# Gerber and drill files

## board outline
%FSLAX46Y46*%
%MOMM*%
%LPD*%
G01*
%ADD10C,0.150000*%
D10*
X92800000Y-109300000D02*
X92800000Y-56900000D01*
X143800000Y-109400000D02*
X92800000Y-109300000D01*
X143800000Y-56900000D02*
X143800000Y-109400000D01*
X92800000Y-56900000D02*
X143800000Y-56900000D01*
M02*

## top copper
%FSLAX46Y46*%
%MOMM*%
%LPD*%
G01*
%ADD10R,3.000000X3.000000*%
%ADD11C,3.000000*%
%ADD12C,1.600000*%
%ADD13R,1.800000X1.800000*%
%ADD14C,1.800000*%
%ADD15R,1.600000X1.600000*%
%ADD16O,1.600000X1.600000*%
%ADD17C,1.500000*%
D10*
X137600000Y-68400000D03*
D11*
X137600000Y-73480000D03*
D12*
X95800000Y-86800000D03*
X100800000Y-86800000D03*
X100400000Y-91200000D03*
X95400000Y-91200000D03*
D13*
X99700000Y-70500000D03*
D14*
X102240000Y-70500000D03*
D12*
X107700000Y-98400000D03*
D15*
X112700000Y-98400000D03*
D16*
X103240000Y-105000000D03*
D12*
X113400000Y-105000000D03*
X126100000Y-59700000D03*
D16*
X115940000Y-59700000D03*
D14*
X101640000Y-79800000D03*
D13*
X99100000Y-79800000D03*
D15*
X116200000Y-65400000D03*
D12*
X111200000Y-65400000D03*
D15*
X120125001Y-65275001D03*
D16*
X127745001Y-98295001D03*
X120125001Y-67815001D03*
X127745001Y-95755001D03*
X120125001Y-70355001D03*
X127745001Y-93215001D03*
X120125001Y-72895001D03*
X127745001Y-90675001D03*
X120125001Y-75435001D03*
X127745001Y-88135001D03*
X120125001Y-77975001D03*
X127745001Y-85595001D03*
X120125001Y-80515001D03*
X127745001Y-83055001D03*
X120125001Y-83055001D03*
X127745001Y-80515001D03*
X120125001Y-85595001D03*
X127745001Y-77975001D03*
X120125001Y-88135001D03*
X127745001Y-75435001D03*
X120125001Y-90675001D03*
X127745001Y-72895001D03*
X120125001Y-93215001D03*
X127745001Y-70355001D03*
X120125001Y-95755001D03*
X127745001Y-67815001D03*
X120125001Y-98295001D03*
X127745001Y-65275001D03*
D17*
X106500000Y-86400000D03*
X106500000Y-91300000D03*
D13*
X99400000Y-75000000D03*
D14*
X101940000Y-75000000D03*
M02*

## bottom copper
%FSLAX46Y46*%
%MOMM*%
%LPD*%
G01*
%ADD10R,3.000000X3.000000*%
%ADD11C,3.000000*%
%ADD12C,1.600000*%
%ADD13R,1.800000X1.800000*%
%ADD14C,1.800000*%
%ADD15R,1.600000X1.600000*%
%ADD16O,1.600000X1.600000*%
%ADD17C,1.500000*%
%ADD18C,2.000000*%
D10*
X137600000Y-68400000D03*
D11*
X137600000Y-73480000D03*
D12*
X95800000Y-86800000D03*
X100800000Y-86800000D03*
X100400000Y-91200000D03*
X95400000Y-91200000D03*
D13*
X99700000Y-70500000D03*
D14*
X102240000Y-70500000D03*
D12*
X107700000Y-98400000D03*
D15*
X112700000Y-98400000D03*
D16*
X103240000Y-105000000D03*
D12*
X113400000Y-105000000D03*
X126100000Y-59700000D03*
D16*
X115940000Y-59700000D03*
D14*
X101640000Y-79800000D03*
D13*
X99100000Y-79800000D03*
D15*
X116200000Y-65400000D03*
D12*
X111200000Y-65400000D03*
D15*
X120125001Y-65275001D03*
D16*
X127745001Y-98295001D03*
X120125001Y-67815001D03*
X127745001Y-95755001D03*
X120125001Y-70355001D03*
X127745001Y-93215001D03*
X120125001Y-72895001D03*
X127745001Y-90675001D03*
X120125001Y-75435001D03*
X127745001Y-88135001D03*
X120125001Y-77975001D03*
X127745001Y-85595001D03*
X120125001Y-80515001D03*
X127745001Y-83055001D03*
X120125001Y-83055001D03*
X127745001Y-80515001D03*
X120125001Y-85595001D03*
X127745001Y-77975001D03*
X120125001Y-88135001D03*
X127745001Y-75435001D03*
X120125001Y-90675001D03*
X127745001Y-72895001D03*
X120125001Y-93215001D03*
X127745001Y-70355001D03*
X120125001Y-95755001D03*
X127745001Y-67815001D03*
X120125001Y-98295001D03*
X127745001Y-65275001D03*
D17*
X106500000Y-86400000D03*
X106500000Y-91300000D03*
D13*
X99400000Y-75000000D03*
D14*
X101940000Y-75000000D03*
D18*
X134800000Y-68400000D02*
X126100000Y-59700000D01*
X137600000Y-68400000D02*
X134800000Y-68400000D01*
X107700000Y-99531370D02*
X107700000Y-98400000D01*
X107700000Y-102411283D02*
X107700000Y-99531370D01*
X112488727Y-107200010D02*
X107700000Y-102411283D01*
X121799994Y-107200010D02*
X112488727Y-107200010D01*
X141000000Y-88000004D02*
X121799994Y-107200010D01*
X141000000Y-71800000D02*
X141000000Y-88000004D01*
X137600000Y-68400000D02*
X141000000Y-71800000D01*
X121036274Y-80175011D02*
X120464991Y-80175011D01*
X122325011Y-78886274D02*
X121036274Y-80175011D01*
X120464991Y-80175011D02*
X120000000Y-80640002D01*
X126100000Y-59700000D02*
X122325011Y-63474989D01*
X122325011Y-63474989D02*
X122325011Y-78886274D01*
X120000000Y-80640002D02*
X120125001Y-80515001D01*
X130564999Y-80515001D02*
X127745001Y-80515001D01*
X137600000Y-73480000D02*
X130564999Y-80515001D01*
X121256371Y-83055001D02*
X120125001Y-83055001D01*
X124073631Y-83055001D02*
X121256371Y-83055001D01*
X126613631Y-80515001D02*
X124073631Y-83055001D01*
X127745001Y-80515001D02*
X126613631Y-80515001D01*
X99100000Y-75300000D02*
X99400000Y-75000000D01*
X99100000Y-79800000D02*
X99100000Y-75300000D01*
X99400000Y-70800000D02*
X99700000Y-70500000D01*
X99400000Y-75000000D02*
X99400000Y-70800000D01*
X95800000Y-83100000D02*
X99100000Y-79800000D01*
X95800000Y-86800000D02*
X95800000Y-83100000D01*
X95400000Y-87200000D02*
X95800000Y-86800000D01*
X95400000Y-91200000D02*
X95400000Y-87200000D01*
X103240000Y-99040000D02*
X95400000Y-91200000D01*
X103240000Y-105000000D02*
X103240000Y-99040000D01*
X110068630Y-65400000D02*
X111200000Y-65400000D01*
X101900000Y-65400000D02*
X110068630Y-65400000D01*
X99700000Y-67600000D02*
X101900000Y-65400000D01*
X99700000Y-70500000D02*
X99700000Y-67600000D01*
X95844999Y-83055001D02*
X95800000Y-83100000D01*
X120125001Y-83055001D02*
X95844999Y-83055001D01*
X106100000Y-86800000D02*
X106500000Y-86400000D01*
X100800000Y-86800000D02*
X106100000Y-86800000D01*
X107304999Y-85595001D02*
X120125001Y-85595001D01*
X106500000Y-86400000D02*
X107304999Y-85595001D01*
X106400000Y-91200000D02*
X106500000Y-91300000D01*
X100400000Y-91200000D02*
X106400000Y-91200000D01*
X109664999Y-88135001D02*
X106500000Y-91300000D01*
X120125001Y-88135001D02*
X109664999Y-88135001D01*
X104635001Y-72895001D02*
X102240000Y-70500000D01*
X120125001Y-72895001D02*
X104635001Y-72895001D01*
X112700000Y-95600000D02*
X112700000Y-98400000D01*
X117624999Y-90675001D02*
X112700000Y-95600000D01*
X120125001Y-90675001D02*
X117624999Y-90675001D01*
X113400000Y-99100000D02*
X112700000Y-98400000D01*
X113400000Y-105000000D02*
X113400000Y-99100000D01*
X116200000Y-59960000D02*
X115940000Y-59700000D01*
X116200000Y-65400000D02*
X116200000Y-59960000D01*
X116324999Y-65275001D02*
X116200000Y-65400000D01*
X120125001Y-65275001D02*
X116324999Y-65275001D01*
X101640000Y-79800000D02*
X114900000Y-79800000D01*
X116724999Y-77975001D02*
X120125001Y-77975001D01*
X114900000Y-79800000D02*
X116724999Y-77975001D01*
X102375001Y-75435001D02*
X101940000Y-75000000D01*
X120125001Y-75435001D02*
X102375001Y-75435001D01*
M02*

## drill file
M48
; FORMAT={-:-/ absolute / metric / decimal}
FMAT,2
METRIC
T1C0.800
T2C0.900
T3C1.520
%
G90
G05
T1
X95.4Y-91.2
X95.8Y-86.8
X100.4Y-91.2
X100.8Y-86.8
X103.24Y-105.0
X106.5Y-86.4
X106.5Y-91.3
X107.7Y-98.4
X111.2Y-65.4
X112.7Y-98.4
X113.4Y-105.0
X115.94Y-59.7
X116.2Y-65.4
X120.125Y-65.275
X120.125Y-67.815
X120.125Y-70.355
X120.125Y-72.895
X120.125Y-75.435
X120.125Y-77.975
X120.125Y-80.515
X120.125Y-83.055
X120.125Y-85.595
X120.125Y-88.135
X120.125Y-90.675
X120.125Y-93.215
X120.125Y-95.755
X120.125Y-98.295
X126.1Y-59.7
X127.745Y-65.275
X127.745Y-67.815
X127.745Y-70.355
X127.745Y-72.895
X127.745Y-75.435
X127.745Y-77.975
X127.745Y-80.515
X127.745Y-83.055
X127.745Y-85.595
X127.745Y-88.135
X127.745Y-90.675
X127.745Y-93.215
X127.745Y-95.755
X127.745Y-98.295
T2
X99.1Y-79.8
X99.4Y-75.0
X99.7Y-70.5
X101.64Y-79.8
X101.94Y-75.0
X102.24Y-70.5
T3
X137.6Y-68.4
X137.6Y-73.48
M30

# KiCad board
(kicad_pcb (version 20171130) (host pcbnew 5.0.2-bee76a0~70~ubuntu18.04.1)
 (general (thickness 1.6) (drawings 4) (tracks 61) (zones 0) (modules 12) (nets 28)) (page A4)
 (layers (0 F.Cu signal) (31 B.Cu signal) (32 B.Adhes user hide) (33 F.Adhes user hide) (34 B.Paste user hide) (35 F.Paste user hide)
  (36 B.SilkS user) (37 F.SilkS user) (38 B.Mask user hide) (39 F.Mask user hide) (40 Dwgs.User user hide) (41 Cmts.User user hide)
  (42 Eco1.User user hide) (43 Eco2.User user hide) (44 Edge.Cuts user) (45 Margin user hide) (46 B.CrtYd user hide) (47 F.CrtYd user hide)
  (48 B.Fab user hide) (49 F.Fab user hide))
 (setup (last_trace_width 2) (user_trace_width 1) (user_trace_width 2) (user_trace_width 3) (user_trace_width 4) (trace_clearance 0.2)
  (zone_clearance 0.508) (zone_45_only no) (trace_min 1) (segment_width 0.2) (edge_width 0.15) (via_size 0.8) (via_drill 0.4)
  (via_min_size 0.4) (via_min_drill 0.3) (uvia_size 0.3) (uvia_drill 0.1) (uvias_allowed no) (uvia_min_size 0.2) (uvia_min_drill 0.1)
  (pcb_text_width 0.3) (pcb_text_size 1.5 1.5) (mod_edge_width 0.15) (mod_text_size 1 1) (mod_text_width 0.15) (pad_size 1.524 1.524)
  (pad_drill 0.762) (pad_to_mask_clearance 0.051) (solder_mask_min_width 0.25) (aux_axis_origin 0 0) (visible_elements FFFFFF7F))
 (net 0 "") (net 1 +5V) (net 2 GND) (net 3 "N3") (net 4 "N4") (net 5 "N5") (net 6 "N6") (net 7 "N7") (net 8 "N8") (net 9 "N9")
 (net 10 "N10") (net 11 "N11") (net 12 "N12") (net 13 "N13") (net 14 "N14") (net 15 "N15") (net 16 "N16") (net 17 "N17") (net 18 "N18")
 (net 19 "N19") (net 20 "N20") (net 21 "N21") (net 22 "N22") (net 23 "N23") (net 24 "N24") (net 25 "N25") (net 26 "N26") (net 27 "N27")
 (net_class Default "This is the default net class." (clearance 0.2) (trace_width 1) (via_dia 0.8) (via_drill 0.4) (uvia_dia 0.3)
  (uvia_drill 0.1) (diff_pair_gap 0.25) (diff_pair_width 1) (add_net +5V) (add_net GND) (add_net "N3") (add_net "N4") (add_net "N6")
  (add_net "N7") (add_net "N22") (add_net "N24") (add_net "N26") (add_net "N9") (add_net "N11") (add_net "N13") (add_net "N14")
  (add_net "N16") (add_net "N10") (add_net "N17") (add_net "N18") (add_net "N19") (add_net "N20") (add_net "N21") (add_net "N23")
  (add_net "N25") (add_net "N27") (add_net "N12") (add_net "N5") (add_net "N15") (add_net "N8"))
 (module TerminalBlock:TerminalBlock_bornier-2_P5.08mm (layer F.Cu) (at 137.6 68.4 270)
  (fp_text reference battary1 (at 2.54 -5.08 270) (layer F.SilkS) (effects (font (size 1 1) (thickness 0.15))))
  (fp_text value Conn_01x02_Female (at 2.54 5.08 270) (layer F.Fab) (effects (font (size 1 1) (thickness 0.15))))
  (pad 1 thru_hole rect (at 0 0 270) (size 3 3) (drill 1.52) (layers *.Cu *.Mask) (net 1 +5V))
  (pad 2 thru_hole circle (at 5.08 0 270) (size 3 3) (drill 1.52) (layers *.Cu *.Mask) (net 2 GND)))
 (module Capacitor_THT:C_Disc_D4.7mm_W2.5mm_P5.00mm (layer F.Cu) (at 95.8 86.8)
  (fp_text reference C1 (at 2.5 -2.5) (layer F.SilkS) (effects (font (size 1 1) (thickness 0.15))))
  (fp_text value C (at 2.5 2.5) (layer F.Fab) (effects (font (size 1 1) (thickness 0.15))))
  (pad 1 thru_hole circle (at 0 0) (size 1.6 1.6) (drill 0.8) (layers *.Cu *.Mask) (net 2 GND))
  (pad 2 thru_hole circle (at 5 0) (size 1.6 1.6) (drill 0.8) (layers *.Cu *.Mask) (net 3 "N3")))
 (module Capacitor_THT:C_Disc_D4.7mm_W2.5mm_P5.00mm (layer F.Cu) (at 95.4 91.2)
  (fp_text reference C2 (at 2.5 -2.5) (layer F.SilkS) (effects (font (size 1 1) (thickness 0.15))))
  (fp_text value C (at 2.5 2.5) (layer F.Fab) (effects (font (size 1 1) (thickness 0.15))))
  (pad 2 thru_hole circle (at 5 0) (size 1.6 1.6) (drill 0.8) (layers *.Cu *.Mask) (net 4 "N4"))
  (pad 1 thru_hole circle (at 0 0) (size 1.6 1.6) (drill 0.8) (layers *.Cu *.Mask) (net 2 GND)))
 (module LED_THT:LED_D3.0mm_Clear (layer F.Cu) (at 99.7 70.5)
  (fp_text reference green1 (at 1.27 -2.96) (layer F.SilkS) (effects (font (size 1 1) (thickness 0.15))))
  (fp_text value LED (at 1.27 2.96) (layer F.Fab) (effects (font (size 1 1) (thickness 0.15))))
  (pad 1 thru_hole rect (at 0 0) (size 1.8 1.8) (drill 0.9) (layers *.Cu *.Mask) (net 2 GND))
  (pad 2 thru_hole circle (at 2.54 0) (size 1.8 1.8) (drill 0.9) (layers *.Cu *.Mask) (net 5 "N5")))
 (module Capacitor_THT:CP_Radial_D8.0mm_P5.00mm (layer F.Cu) (at 112.7 98.4 180)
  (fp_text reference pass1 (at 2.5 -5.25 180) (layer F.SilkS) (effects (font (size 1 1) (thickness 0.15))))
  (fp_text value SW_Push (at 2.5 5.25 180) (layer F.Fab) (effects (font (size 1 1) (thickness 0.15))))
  (pad 2 thru_hole circle (at 5 0 180) (size 1.6 1.6) (drill 0.8) (layers *.Cu *.Mask) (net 1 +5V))
  (pad 1 thru_hole rect (at 0 0 180) (size 1.6 1.6) (drill 0.8) (layers *.Cu *.Mask) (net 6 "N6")))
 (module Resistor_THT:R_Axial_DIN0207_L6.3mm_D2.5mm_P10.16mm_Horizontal (layer F.Cu) (at 113.4 105 180)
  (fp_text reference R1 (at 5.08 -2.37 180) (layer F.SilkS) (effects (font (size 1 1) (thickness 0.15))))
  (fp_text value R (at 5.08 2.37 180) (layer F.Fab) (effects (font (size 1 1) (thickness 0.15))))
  (pad 2 thru_hole oval (at 10.16 0 180) (size 1.6 1.6) (drill 0.8) (layers *.Cu *.Mask) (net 2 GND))
  (pad 1 thru_hole circle (at 0 0 180) (size 1.6 1.6) (drill 0.8) (layers *.Cu *.Mask) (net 6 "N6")))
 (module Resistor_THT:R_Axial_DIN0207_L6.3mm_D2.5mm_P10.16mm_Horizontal (layer F.Cu) (at 126.1 59.7 180)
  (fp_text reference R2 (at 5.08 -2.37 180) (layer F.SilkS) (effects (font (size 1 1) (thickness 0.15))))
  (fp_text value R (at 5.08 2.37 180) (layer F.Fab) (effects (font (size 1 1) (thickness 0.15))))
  (pad 1 thru_hole circle (at 0 0 180) (size 1.6 1.6) (drill 0.8) (layers *.Cu *.Mask) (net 1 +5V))
  (pad 2 thru_hole oval (at 10.16 0 180) (size 1.6 1.6) (drill 0.8) (layers *.Cu *.Mask) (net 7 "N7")))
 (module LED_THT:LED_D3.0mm (layer F.Cu) (at 99.1 79.8)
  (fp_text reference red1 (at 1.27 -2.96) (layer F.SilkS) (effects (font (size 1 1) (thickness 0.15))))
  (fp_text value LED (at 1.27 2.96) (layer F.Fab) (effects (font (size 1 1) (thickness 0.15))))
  (pad 2 thru_hole circle (at 2.54 0) (size 1.8 1.8) (drill 0.9) (layers *.Cu *.Mask) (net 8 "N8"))
  (pad 1 thru_hole rect (at 0 0) (size 1.8 1.8) (drill 0.9) (layers *.Cu *.Mask) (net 2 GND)))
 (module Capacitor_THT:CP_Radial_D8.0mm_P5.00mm (layer F.Cu) (at 116.2 65.4 180)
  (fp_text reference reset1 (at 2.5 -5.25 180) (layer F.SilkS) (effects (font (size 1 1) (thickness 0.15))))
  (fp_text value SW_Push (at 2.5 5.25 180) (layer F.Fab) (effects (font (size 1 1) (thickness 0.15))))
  (pad 1 thru_hole rect (at 0 0 180) (size 1.6 1.6) (drill 0.8) (layers *.Cu *.Mask) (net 7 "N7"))
  (pad 2 thru_hole circle (at 5 0 180) (size 1.6 1.6) (drill 0.8) (layers *.Cu *.Mask) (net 2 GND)))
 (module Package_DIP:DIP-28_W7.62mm (layer F.Cu) (at 120.125001 65.275001)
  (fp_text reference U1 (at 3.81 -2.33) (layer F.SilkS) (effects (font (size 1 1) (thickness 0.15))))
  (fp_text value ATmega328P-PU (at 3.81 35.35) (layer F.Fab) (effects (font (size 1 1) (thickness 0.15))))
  (pad 1 thru_hole rect (at 0 0) (size 1.6 1.6) (drill 0.8) (layers *.Cu *.Mask) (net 7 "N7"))
  (pad 15 thru_hole oval (at 7.62 33.02) (size 1.6 1.6) (drill 0.8) (layers *.Cu *.Mask) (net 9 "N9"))
  (pad 2 thru_hole oval (at 0 2.54) (size 1.6 1.6) (drill 0.8) (layers *.Cu *.Mask) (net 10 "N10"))
  (pad 16 thru_hole oval (at 7.62 30.48) (size 1.6 1.6) (drill 0.8) (layers *.Cu *.Mask) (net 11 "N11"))
  (pad 3 thru_hole oval (at 0 5.08) (size 1.6 1.6) (drill 0.8) (layers *.Cu *.Mask) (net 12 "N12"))
  (pad 17 thru_hole oval (at 7.62 27.94) (size 1.6 1.6) (drill 0.8) (layers *.Cu *.Mask) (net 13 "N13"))
  (pad 4 thru_hole oval (at 0 7.62) (size 1.6 1.6) (drill 0.8) (layers *.Cu *.Mask) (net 5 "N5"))
  (pad 18 thru_hole oval (at 7.62 25.4) (size 1.6 1.6) (drill 0.8) (layers *.Cu *.Mask) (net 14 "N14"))
  (pad 5 thru_hole oval (at 0 10.16) (size 1.6 1.6) (drill 0.8) (layers *.Cu *.Mask) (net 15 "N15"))
  (pad 19 thru_hole oval (at 7.62 22.86) (size 1.6 1.6) (drill 0.8) (layers *.Cu *.Mask) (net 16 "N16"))
  (pad 6 thru_hole oval (at 0 12.7) (size 1.6 1.6) (drill 0.8) (layers *.Cu *.Mask) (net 8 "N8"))
  (pad 20 thru_hole oval (at 7.62 20.32) (size 1.6 1.6) (drill 0.8) (layers *.Cu *.Mask) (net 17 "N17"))
  (pad 7 thru_hole oval (at 0 15.24) (size 1.6 1.6) (drill 0.8) (layers *.Cu *.Mask) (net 1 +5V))
  (pad 21 thru_hole oval (at 7.62 17.78) (size 1.6 1.6) (drill 0.8) (layers *.Cu *.Mask) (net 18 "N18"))
  (pad 8 thru_hole oval (at 0 17.78) (size 1.6 1.6) (drill 0.8) (layers *.Cu *.Mask) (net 2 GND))
  (pad 22 thru_hole oval (at 7.62 15.24) (size 1.6 1.6) (drill 0.8) (layers *.Cu *.Mask) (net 2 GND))
  (pad 9 thru_hole oval (at 0 20.32) (size 1.6 1.6) (drill 0.8) (layers *.Cu *.Mask) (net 3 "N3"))
  (pad 23 thru_hole oval (at 7.62 12.7) (size 1.6 1.6) (drill 0.8) (layers *.Cu *.Mask) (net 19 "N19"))
  (pad 10 thru_hole oval (at 0 22.86) (size 1.6 1.6) (drill 0.8) (layers *.Cu *.Mask) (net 4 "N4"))
  (pad 24 thru_hole oval (at 7.62 10.16) (size 1.6 1.6) (drill 0.8) (layers *.Cu *.Mask) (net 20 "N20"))
  (pad 11 thru_hole oval (at 0 25.4) (size 1.6 1.6) (drill 0.8) (layers *.Cu *.Mask) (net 6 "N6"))
  (pad 25 thru_hole oval (at 7.62 7.62) (size 1.6 1.6) (drill 0.8) (layers *.Cu *.Mask) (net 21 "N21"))
  (pad 12 thru_hole oval (at 0 27.94) (size 1.6 1.6) (drill 0.8) (layers *.Cu *.Mask) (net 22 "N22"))
  (pad 26 thru_hole oval (at 7.62 5.08) (size 1.6 1.6) (drill 0.8) (layers *.Cu *.Mask) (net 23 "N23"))
  (pad 13 thru_hole oval (at 0 30.48) (size 1.6 1.6) (drill 0.8) (layers *.Cu *.Mask) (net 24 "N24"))
  (pad 27 thru_hole oval (at 7.62 2.54) (size 1.6 1.6) (drill 0.8) (layers *.Cu *.Mask) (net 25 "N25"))
  (pad 14 thru_hole oval (at 0 33.02) (size 1.6 1.6) (drill 0.8) (layers *.Cu *.Mask) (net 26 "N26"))
  (pad 28 thru_hole oval (at 7.62 0) (size 1.6 1.6) (drill 0.8) (layers *.Cu *.Mask) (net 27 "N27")))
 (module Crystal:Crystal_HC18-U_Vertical (layer F.Cu) (at 106.5 86.4 270)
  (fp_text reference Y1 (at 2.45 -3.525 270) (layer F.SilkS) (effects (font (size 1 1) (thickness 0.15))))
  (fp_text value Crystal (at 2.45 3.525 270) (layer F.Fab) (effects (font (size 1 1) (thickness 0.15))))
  (pad 1 thru_hole circle (at 0 0 270) (size 1.5 1.5) (drill 0.8) (layers *.Cu *.Mask) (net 3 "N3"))
  (pad 2 thru_hole circle (at 4.9 0 270) (size 1.5 1.5) (drill 0.8) (layers *.Cu *.Mask) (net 4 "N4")))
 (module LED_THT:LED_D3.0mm (layer F.Cu) (at 99.4 75)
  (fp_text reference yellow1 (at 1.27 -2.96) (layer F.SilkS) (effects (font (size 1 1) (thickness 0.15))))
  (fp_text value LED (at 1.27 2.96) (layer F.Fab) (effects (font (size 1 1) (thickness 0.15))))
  (pad 1 thru_hole rect (at 0 0) (size 1.8 1.8) (drill 0.9) (layers *.Cu *.Mask) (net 2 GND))
  (pad 2 thru_hole circle (at 2.54 0) (size 1.8 1.8) (drill 0.9) (layers *.Cu *.Mask) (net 15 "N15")))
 (gr_line (start 92.8 109.3) (end 92.8 56.9) (layer Edge.Cuts) (width 0.15))
 (gr_line (start 143.8 109.4) (end 92.8 109.3) (layer Edge.Cuts) (width 0.15))
 (gr_line (start 143.8 56.9) (end 143.8 109.4) (layer Edge.Cuts) (width 0.15))
 (gr_line (start 92.8 56.9) (end 143.8 56.9) (layer Edge.Cuts) (width 0.15))
 (segment (start 134.8 68.4) (end 126.1 59.7) (width 2) (layer B.Cu) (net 1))
 (segment (start 137.6 68.4) (end 134.8 68.4) (width 2) (layer B.Cu) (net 1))
 (segment (start 107.7 99.53137) (end 107.7 98.4) (width 2) (layer B.Cu) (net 1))
 (segment (start 107.7 102.411283) (end 107.7 99.53137) (width 2) (layer B.Cu) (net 1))
 (segment (start 112.488727 107.20001) (end 107.7 102.411283) (width 2) (layer B.Cu) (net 1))
 (segment (start 121.799994 107.20001) (end 112.488727 107.20001) (width 2) (layer B.Cu) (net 1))
 (segment (start 141 88.000004) (end 121.799994 107.20001) (width 2) (layer B.Cu) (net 1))
 (segment (start 141 71.8) (end 141 88.000004) (width 2) (layer B.Cu) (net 1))
 (segment (start 137.6 68.4) (end 141 71.8) (width 2) (layer B.Cu) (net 1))
 (segment (start 121.036274 80.175011) (end 120.464991 80.175011) (width 2) (layer B.Cu) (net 1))
 (segment (start 122.325011 78.886274) (end 121.036274 80.175011) (width 2) (layer B.Cu) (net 1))
 (segment (start 120.464991 80.175011) (end 120 80.640002) (width 2) (layer B.Cu) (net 1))
 (segment (start 126.1 59.7) (end 122.325011 63.474989) (width 2) (layer B.Cu) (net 1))
 (segment (start 122.325011 63.474989) (end 122.325011 78.886274) (width 2) (layer B.Cu) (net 1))
 (segment (start 120 80.640002) (end 120.125001 80.515001) (width 2) (layer B.Cu) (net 1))
 (segment (start 130.564999 80.515001) (end 127.745001 80.515001) (width 2) (layer B.Cu) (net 2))
 (segment (start 137.6 73.48) (end 130.564999 80.515001) (width 2) (layer B.Cu) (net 2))
 (segment (start 121.256371 83.055001) (end 120.125001 83.055001) (width 2) (layer B.Cu) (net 2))
 (segment (start 124.073631 83.055001) (end 121.256371 83.055001) (width 2) (layer B.Cu) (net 2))
 (segment (start 126.613631 80.515001) (end 124.073631 83.055001) (width 2) (layer B.Cu) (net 2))
 (segment (start 127.745001 80.515001) (end 126.613631 80.515001) (width 2) (layer B.Cu) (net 2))
 (segment (start 99.1 75.3) (end 99.4 75) (width 2) (layer B.Cu) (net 2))
 (segment (start 99.1 79.8) (end 99.1 75.3) (width 2) (layer B.Cu) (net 2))
 (segment (start 99.4 70.8) (end 99.7 70.5) (width 2) (layer B.Cu) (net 2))
 (segment (start 99.4 75) (end 99.4 70.8) (width 2) (layer B.Cu) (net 2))
 (segment (start 95.8 83.1) (end 99.1 79.8) (width 2) (layer B.Cu) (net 2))
 (segment (start 95.8 86.8) (end 95.8 83.1) (width 2) (layer B.Cu) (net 2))
 (segment (start 95.4 87.2) (end 95.8 86.8) (width 2) (layer B.Cu) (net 2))
 (segment (start 95.4 91.2) (end 95.4 87.2) (width 2) (layer B.Cu) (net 2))
 (segment (start 103.24 99.04) (end 95.4 91.2) (width 2) (layer B.Cu) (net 2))
 (segment (start 103.24 105) (end 103.24 99.04) (width 2) (layer B.Cu) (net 2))
 (segment (start 110.06863 65.4) (end 111.2 65.4) (width 2) (layer B.Cu) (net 2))
 (segment (start 101.9 65.4) (end 110.06863 65.4) (width 2) (layer B.Cu) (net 2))
 (segment (start 99.7 67.6) (end 101.9 65.4) (width 2) (layer B.Cu) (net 2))
 (segment (start 99.7 70.5) (end 99.7 67.6) (width 2) (layer B.Cu) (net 2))
 (segment (start 95.844999 83.055001) (end 95.8 83.1) (width 2) (layer B.Cu) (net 2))
 (segment (start 120.125001 83.055001) (end 95.844999 83.055001) (width 2) (layer B.Cu) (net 2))
 (segment (start 106.1 86.8) (end 106.5 86.4) (width 2) (layer B.Cu) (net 3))
 (segment (start 100.8 86.8) (end 106.1 86.8) (width 2) (layer B.Cu) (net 3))
 (segment (start 107.304999 85.595001) (end 120.125001 85.595001) (width 2) (layer B.Cu) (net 3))
 (segment (start 106.5 86.4) (end 107.304999 85.595001) (width 2) (layer B.Cu) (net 3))
 (segment (start 106.4 91.2) (end 106.5 91.3) (width 2) (layer B.Cu) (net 4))
 (segment (start 100.4 91.2) (end 106.4 91.2) (width 2) (layer B.Cu) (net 4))
 (segment (start 109.664999 88.135001) (end 106.5 91.3) (width 2) (layer B.Cu) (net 4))
 (segment (start 120.125001 88.135001) (end 109.664999 88.135001) (width 2) (layer B.Cu) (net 4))
 (segment (start 104.635001 72.895001) (end 102.24 70.5) (width 2) (layer B.Cu) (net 5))
 (segment (start 120.125001 72.895001) (end 104.635001 72.895001) (width 2) (layer B.Cu) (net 5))
 (segment (start 112.7 95.6) (end 112.7 98.4) (width 2) (layer B.Cu) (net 6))
 (segment (start 117.624999 90.675001) (end 112.7 95.6) (width 2) (layer B.Cu) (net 6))
 (segment (start 120.125001 90.675001) (end 117.624999 90.675001) (width 2) (layer B.Cu) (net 6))
 (segment (start 113.4 99.1) (end 112.7 98.4) (width 2) (layer B.Cu) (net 6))
 (segment (start 113.4 105) (end 113.4 99.1) (width 2) (layer B.Cu) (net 6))
 (segment (start 116.2 59.96) (end 115.94 59.7) (width 2) (layer B.Cu) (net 7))
 (segment (start 116.2 65.4) (end 116.2 59.96) (width 2) (layer B.Cu) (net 7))
 (segment (start 116.324999 65.275001) (end 116.2 65.4) (width 2) (layer B.Cu) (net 7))
 (segment (start 120.125001 65.275001) (end 116.324999 65.275001) (width 2) (layer B.Cu) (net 7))
 (segment (start 101.64 79.8) (end 114.9 79.8) (width 2) (layer B.Cu) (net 8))
 (segment (start 116.724999 77.975001) (end 120.125001 77.975001) (width 2) (layer B.Cu) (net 8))
 (segment (start 114.9 79.8) (end 116.724999 77.975001) (width 2) (layer B.Cu) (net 8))
 (segment (start 102.375001 75.435001) (end 101.94 75) (width 2) (layer B.Cu) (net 15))
 (segment (start 120.125001 75.435001) (end 102.375001 75.435001) (width 2) (layer B.Cu) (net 15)))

